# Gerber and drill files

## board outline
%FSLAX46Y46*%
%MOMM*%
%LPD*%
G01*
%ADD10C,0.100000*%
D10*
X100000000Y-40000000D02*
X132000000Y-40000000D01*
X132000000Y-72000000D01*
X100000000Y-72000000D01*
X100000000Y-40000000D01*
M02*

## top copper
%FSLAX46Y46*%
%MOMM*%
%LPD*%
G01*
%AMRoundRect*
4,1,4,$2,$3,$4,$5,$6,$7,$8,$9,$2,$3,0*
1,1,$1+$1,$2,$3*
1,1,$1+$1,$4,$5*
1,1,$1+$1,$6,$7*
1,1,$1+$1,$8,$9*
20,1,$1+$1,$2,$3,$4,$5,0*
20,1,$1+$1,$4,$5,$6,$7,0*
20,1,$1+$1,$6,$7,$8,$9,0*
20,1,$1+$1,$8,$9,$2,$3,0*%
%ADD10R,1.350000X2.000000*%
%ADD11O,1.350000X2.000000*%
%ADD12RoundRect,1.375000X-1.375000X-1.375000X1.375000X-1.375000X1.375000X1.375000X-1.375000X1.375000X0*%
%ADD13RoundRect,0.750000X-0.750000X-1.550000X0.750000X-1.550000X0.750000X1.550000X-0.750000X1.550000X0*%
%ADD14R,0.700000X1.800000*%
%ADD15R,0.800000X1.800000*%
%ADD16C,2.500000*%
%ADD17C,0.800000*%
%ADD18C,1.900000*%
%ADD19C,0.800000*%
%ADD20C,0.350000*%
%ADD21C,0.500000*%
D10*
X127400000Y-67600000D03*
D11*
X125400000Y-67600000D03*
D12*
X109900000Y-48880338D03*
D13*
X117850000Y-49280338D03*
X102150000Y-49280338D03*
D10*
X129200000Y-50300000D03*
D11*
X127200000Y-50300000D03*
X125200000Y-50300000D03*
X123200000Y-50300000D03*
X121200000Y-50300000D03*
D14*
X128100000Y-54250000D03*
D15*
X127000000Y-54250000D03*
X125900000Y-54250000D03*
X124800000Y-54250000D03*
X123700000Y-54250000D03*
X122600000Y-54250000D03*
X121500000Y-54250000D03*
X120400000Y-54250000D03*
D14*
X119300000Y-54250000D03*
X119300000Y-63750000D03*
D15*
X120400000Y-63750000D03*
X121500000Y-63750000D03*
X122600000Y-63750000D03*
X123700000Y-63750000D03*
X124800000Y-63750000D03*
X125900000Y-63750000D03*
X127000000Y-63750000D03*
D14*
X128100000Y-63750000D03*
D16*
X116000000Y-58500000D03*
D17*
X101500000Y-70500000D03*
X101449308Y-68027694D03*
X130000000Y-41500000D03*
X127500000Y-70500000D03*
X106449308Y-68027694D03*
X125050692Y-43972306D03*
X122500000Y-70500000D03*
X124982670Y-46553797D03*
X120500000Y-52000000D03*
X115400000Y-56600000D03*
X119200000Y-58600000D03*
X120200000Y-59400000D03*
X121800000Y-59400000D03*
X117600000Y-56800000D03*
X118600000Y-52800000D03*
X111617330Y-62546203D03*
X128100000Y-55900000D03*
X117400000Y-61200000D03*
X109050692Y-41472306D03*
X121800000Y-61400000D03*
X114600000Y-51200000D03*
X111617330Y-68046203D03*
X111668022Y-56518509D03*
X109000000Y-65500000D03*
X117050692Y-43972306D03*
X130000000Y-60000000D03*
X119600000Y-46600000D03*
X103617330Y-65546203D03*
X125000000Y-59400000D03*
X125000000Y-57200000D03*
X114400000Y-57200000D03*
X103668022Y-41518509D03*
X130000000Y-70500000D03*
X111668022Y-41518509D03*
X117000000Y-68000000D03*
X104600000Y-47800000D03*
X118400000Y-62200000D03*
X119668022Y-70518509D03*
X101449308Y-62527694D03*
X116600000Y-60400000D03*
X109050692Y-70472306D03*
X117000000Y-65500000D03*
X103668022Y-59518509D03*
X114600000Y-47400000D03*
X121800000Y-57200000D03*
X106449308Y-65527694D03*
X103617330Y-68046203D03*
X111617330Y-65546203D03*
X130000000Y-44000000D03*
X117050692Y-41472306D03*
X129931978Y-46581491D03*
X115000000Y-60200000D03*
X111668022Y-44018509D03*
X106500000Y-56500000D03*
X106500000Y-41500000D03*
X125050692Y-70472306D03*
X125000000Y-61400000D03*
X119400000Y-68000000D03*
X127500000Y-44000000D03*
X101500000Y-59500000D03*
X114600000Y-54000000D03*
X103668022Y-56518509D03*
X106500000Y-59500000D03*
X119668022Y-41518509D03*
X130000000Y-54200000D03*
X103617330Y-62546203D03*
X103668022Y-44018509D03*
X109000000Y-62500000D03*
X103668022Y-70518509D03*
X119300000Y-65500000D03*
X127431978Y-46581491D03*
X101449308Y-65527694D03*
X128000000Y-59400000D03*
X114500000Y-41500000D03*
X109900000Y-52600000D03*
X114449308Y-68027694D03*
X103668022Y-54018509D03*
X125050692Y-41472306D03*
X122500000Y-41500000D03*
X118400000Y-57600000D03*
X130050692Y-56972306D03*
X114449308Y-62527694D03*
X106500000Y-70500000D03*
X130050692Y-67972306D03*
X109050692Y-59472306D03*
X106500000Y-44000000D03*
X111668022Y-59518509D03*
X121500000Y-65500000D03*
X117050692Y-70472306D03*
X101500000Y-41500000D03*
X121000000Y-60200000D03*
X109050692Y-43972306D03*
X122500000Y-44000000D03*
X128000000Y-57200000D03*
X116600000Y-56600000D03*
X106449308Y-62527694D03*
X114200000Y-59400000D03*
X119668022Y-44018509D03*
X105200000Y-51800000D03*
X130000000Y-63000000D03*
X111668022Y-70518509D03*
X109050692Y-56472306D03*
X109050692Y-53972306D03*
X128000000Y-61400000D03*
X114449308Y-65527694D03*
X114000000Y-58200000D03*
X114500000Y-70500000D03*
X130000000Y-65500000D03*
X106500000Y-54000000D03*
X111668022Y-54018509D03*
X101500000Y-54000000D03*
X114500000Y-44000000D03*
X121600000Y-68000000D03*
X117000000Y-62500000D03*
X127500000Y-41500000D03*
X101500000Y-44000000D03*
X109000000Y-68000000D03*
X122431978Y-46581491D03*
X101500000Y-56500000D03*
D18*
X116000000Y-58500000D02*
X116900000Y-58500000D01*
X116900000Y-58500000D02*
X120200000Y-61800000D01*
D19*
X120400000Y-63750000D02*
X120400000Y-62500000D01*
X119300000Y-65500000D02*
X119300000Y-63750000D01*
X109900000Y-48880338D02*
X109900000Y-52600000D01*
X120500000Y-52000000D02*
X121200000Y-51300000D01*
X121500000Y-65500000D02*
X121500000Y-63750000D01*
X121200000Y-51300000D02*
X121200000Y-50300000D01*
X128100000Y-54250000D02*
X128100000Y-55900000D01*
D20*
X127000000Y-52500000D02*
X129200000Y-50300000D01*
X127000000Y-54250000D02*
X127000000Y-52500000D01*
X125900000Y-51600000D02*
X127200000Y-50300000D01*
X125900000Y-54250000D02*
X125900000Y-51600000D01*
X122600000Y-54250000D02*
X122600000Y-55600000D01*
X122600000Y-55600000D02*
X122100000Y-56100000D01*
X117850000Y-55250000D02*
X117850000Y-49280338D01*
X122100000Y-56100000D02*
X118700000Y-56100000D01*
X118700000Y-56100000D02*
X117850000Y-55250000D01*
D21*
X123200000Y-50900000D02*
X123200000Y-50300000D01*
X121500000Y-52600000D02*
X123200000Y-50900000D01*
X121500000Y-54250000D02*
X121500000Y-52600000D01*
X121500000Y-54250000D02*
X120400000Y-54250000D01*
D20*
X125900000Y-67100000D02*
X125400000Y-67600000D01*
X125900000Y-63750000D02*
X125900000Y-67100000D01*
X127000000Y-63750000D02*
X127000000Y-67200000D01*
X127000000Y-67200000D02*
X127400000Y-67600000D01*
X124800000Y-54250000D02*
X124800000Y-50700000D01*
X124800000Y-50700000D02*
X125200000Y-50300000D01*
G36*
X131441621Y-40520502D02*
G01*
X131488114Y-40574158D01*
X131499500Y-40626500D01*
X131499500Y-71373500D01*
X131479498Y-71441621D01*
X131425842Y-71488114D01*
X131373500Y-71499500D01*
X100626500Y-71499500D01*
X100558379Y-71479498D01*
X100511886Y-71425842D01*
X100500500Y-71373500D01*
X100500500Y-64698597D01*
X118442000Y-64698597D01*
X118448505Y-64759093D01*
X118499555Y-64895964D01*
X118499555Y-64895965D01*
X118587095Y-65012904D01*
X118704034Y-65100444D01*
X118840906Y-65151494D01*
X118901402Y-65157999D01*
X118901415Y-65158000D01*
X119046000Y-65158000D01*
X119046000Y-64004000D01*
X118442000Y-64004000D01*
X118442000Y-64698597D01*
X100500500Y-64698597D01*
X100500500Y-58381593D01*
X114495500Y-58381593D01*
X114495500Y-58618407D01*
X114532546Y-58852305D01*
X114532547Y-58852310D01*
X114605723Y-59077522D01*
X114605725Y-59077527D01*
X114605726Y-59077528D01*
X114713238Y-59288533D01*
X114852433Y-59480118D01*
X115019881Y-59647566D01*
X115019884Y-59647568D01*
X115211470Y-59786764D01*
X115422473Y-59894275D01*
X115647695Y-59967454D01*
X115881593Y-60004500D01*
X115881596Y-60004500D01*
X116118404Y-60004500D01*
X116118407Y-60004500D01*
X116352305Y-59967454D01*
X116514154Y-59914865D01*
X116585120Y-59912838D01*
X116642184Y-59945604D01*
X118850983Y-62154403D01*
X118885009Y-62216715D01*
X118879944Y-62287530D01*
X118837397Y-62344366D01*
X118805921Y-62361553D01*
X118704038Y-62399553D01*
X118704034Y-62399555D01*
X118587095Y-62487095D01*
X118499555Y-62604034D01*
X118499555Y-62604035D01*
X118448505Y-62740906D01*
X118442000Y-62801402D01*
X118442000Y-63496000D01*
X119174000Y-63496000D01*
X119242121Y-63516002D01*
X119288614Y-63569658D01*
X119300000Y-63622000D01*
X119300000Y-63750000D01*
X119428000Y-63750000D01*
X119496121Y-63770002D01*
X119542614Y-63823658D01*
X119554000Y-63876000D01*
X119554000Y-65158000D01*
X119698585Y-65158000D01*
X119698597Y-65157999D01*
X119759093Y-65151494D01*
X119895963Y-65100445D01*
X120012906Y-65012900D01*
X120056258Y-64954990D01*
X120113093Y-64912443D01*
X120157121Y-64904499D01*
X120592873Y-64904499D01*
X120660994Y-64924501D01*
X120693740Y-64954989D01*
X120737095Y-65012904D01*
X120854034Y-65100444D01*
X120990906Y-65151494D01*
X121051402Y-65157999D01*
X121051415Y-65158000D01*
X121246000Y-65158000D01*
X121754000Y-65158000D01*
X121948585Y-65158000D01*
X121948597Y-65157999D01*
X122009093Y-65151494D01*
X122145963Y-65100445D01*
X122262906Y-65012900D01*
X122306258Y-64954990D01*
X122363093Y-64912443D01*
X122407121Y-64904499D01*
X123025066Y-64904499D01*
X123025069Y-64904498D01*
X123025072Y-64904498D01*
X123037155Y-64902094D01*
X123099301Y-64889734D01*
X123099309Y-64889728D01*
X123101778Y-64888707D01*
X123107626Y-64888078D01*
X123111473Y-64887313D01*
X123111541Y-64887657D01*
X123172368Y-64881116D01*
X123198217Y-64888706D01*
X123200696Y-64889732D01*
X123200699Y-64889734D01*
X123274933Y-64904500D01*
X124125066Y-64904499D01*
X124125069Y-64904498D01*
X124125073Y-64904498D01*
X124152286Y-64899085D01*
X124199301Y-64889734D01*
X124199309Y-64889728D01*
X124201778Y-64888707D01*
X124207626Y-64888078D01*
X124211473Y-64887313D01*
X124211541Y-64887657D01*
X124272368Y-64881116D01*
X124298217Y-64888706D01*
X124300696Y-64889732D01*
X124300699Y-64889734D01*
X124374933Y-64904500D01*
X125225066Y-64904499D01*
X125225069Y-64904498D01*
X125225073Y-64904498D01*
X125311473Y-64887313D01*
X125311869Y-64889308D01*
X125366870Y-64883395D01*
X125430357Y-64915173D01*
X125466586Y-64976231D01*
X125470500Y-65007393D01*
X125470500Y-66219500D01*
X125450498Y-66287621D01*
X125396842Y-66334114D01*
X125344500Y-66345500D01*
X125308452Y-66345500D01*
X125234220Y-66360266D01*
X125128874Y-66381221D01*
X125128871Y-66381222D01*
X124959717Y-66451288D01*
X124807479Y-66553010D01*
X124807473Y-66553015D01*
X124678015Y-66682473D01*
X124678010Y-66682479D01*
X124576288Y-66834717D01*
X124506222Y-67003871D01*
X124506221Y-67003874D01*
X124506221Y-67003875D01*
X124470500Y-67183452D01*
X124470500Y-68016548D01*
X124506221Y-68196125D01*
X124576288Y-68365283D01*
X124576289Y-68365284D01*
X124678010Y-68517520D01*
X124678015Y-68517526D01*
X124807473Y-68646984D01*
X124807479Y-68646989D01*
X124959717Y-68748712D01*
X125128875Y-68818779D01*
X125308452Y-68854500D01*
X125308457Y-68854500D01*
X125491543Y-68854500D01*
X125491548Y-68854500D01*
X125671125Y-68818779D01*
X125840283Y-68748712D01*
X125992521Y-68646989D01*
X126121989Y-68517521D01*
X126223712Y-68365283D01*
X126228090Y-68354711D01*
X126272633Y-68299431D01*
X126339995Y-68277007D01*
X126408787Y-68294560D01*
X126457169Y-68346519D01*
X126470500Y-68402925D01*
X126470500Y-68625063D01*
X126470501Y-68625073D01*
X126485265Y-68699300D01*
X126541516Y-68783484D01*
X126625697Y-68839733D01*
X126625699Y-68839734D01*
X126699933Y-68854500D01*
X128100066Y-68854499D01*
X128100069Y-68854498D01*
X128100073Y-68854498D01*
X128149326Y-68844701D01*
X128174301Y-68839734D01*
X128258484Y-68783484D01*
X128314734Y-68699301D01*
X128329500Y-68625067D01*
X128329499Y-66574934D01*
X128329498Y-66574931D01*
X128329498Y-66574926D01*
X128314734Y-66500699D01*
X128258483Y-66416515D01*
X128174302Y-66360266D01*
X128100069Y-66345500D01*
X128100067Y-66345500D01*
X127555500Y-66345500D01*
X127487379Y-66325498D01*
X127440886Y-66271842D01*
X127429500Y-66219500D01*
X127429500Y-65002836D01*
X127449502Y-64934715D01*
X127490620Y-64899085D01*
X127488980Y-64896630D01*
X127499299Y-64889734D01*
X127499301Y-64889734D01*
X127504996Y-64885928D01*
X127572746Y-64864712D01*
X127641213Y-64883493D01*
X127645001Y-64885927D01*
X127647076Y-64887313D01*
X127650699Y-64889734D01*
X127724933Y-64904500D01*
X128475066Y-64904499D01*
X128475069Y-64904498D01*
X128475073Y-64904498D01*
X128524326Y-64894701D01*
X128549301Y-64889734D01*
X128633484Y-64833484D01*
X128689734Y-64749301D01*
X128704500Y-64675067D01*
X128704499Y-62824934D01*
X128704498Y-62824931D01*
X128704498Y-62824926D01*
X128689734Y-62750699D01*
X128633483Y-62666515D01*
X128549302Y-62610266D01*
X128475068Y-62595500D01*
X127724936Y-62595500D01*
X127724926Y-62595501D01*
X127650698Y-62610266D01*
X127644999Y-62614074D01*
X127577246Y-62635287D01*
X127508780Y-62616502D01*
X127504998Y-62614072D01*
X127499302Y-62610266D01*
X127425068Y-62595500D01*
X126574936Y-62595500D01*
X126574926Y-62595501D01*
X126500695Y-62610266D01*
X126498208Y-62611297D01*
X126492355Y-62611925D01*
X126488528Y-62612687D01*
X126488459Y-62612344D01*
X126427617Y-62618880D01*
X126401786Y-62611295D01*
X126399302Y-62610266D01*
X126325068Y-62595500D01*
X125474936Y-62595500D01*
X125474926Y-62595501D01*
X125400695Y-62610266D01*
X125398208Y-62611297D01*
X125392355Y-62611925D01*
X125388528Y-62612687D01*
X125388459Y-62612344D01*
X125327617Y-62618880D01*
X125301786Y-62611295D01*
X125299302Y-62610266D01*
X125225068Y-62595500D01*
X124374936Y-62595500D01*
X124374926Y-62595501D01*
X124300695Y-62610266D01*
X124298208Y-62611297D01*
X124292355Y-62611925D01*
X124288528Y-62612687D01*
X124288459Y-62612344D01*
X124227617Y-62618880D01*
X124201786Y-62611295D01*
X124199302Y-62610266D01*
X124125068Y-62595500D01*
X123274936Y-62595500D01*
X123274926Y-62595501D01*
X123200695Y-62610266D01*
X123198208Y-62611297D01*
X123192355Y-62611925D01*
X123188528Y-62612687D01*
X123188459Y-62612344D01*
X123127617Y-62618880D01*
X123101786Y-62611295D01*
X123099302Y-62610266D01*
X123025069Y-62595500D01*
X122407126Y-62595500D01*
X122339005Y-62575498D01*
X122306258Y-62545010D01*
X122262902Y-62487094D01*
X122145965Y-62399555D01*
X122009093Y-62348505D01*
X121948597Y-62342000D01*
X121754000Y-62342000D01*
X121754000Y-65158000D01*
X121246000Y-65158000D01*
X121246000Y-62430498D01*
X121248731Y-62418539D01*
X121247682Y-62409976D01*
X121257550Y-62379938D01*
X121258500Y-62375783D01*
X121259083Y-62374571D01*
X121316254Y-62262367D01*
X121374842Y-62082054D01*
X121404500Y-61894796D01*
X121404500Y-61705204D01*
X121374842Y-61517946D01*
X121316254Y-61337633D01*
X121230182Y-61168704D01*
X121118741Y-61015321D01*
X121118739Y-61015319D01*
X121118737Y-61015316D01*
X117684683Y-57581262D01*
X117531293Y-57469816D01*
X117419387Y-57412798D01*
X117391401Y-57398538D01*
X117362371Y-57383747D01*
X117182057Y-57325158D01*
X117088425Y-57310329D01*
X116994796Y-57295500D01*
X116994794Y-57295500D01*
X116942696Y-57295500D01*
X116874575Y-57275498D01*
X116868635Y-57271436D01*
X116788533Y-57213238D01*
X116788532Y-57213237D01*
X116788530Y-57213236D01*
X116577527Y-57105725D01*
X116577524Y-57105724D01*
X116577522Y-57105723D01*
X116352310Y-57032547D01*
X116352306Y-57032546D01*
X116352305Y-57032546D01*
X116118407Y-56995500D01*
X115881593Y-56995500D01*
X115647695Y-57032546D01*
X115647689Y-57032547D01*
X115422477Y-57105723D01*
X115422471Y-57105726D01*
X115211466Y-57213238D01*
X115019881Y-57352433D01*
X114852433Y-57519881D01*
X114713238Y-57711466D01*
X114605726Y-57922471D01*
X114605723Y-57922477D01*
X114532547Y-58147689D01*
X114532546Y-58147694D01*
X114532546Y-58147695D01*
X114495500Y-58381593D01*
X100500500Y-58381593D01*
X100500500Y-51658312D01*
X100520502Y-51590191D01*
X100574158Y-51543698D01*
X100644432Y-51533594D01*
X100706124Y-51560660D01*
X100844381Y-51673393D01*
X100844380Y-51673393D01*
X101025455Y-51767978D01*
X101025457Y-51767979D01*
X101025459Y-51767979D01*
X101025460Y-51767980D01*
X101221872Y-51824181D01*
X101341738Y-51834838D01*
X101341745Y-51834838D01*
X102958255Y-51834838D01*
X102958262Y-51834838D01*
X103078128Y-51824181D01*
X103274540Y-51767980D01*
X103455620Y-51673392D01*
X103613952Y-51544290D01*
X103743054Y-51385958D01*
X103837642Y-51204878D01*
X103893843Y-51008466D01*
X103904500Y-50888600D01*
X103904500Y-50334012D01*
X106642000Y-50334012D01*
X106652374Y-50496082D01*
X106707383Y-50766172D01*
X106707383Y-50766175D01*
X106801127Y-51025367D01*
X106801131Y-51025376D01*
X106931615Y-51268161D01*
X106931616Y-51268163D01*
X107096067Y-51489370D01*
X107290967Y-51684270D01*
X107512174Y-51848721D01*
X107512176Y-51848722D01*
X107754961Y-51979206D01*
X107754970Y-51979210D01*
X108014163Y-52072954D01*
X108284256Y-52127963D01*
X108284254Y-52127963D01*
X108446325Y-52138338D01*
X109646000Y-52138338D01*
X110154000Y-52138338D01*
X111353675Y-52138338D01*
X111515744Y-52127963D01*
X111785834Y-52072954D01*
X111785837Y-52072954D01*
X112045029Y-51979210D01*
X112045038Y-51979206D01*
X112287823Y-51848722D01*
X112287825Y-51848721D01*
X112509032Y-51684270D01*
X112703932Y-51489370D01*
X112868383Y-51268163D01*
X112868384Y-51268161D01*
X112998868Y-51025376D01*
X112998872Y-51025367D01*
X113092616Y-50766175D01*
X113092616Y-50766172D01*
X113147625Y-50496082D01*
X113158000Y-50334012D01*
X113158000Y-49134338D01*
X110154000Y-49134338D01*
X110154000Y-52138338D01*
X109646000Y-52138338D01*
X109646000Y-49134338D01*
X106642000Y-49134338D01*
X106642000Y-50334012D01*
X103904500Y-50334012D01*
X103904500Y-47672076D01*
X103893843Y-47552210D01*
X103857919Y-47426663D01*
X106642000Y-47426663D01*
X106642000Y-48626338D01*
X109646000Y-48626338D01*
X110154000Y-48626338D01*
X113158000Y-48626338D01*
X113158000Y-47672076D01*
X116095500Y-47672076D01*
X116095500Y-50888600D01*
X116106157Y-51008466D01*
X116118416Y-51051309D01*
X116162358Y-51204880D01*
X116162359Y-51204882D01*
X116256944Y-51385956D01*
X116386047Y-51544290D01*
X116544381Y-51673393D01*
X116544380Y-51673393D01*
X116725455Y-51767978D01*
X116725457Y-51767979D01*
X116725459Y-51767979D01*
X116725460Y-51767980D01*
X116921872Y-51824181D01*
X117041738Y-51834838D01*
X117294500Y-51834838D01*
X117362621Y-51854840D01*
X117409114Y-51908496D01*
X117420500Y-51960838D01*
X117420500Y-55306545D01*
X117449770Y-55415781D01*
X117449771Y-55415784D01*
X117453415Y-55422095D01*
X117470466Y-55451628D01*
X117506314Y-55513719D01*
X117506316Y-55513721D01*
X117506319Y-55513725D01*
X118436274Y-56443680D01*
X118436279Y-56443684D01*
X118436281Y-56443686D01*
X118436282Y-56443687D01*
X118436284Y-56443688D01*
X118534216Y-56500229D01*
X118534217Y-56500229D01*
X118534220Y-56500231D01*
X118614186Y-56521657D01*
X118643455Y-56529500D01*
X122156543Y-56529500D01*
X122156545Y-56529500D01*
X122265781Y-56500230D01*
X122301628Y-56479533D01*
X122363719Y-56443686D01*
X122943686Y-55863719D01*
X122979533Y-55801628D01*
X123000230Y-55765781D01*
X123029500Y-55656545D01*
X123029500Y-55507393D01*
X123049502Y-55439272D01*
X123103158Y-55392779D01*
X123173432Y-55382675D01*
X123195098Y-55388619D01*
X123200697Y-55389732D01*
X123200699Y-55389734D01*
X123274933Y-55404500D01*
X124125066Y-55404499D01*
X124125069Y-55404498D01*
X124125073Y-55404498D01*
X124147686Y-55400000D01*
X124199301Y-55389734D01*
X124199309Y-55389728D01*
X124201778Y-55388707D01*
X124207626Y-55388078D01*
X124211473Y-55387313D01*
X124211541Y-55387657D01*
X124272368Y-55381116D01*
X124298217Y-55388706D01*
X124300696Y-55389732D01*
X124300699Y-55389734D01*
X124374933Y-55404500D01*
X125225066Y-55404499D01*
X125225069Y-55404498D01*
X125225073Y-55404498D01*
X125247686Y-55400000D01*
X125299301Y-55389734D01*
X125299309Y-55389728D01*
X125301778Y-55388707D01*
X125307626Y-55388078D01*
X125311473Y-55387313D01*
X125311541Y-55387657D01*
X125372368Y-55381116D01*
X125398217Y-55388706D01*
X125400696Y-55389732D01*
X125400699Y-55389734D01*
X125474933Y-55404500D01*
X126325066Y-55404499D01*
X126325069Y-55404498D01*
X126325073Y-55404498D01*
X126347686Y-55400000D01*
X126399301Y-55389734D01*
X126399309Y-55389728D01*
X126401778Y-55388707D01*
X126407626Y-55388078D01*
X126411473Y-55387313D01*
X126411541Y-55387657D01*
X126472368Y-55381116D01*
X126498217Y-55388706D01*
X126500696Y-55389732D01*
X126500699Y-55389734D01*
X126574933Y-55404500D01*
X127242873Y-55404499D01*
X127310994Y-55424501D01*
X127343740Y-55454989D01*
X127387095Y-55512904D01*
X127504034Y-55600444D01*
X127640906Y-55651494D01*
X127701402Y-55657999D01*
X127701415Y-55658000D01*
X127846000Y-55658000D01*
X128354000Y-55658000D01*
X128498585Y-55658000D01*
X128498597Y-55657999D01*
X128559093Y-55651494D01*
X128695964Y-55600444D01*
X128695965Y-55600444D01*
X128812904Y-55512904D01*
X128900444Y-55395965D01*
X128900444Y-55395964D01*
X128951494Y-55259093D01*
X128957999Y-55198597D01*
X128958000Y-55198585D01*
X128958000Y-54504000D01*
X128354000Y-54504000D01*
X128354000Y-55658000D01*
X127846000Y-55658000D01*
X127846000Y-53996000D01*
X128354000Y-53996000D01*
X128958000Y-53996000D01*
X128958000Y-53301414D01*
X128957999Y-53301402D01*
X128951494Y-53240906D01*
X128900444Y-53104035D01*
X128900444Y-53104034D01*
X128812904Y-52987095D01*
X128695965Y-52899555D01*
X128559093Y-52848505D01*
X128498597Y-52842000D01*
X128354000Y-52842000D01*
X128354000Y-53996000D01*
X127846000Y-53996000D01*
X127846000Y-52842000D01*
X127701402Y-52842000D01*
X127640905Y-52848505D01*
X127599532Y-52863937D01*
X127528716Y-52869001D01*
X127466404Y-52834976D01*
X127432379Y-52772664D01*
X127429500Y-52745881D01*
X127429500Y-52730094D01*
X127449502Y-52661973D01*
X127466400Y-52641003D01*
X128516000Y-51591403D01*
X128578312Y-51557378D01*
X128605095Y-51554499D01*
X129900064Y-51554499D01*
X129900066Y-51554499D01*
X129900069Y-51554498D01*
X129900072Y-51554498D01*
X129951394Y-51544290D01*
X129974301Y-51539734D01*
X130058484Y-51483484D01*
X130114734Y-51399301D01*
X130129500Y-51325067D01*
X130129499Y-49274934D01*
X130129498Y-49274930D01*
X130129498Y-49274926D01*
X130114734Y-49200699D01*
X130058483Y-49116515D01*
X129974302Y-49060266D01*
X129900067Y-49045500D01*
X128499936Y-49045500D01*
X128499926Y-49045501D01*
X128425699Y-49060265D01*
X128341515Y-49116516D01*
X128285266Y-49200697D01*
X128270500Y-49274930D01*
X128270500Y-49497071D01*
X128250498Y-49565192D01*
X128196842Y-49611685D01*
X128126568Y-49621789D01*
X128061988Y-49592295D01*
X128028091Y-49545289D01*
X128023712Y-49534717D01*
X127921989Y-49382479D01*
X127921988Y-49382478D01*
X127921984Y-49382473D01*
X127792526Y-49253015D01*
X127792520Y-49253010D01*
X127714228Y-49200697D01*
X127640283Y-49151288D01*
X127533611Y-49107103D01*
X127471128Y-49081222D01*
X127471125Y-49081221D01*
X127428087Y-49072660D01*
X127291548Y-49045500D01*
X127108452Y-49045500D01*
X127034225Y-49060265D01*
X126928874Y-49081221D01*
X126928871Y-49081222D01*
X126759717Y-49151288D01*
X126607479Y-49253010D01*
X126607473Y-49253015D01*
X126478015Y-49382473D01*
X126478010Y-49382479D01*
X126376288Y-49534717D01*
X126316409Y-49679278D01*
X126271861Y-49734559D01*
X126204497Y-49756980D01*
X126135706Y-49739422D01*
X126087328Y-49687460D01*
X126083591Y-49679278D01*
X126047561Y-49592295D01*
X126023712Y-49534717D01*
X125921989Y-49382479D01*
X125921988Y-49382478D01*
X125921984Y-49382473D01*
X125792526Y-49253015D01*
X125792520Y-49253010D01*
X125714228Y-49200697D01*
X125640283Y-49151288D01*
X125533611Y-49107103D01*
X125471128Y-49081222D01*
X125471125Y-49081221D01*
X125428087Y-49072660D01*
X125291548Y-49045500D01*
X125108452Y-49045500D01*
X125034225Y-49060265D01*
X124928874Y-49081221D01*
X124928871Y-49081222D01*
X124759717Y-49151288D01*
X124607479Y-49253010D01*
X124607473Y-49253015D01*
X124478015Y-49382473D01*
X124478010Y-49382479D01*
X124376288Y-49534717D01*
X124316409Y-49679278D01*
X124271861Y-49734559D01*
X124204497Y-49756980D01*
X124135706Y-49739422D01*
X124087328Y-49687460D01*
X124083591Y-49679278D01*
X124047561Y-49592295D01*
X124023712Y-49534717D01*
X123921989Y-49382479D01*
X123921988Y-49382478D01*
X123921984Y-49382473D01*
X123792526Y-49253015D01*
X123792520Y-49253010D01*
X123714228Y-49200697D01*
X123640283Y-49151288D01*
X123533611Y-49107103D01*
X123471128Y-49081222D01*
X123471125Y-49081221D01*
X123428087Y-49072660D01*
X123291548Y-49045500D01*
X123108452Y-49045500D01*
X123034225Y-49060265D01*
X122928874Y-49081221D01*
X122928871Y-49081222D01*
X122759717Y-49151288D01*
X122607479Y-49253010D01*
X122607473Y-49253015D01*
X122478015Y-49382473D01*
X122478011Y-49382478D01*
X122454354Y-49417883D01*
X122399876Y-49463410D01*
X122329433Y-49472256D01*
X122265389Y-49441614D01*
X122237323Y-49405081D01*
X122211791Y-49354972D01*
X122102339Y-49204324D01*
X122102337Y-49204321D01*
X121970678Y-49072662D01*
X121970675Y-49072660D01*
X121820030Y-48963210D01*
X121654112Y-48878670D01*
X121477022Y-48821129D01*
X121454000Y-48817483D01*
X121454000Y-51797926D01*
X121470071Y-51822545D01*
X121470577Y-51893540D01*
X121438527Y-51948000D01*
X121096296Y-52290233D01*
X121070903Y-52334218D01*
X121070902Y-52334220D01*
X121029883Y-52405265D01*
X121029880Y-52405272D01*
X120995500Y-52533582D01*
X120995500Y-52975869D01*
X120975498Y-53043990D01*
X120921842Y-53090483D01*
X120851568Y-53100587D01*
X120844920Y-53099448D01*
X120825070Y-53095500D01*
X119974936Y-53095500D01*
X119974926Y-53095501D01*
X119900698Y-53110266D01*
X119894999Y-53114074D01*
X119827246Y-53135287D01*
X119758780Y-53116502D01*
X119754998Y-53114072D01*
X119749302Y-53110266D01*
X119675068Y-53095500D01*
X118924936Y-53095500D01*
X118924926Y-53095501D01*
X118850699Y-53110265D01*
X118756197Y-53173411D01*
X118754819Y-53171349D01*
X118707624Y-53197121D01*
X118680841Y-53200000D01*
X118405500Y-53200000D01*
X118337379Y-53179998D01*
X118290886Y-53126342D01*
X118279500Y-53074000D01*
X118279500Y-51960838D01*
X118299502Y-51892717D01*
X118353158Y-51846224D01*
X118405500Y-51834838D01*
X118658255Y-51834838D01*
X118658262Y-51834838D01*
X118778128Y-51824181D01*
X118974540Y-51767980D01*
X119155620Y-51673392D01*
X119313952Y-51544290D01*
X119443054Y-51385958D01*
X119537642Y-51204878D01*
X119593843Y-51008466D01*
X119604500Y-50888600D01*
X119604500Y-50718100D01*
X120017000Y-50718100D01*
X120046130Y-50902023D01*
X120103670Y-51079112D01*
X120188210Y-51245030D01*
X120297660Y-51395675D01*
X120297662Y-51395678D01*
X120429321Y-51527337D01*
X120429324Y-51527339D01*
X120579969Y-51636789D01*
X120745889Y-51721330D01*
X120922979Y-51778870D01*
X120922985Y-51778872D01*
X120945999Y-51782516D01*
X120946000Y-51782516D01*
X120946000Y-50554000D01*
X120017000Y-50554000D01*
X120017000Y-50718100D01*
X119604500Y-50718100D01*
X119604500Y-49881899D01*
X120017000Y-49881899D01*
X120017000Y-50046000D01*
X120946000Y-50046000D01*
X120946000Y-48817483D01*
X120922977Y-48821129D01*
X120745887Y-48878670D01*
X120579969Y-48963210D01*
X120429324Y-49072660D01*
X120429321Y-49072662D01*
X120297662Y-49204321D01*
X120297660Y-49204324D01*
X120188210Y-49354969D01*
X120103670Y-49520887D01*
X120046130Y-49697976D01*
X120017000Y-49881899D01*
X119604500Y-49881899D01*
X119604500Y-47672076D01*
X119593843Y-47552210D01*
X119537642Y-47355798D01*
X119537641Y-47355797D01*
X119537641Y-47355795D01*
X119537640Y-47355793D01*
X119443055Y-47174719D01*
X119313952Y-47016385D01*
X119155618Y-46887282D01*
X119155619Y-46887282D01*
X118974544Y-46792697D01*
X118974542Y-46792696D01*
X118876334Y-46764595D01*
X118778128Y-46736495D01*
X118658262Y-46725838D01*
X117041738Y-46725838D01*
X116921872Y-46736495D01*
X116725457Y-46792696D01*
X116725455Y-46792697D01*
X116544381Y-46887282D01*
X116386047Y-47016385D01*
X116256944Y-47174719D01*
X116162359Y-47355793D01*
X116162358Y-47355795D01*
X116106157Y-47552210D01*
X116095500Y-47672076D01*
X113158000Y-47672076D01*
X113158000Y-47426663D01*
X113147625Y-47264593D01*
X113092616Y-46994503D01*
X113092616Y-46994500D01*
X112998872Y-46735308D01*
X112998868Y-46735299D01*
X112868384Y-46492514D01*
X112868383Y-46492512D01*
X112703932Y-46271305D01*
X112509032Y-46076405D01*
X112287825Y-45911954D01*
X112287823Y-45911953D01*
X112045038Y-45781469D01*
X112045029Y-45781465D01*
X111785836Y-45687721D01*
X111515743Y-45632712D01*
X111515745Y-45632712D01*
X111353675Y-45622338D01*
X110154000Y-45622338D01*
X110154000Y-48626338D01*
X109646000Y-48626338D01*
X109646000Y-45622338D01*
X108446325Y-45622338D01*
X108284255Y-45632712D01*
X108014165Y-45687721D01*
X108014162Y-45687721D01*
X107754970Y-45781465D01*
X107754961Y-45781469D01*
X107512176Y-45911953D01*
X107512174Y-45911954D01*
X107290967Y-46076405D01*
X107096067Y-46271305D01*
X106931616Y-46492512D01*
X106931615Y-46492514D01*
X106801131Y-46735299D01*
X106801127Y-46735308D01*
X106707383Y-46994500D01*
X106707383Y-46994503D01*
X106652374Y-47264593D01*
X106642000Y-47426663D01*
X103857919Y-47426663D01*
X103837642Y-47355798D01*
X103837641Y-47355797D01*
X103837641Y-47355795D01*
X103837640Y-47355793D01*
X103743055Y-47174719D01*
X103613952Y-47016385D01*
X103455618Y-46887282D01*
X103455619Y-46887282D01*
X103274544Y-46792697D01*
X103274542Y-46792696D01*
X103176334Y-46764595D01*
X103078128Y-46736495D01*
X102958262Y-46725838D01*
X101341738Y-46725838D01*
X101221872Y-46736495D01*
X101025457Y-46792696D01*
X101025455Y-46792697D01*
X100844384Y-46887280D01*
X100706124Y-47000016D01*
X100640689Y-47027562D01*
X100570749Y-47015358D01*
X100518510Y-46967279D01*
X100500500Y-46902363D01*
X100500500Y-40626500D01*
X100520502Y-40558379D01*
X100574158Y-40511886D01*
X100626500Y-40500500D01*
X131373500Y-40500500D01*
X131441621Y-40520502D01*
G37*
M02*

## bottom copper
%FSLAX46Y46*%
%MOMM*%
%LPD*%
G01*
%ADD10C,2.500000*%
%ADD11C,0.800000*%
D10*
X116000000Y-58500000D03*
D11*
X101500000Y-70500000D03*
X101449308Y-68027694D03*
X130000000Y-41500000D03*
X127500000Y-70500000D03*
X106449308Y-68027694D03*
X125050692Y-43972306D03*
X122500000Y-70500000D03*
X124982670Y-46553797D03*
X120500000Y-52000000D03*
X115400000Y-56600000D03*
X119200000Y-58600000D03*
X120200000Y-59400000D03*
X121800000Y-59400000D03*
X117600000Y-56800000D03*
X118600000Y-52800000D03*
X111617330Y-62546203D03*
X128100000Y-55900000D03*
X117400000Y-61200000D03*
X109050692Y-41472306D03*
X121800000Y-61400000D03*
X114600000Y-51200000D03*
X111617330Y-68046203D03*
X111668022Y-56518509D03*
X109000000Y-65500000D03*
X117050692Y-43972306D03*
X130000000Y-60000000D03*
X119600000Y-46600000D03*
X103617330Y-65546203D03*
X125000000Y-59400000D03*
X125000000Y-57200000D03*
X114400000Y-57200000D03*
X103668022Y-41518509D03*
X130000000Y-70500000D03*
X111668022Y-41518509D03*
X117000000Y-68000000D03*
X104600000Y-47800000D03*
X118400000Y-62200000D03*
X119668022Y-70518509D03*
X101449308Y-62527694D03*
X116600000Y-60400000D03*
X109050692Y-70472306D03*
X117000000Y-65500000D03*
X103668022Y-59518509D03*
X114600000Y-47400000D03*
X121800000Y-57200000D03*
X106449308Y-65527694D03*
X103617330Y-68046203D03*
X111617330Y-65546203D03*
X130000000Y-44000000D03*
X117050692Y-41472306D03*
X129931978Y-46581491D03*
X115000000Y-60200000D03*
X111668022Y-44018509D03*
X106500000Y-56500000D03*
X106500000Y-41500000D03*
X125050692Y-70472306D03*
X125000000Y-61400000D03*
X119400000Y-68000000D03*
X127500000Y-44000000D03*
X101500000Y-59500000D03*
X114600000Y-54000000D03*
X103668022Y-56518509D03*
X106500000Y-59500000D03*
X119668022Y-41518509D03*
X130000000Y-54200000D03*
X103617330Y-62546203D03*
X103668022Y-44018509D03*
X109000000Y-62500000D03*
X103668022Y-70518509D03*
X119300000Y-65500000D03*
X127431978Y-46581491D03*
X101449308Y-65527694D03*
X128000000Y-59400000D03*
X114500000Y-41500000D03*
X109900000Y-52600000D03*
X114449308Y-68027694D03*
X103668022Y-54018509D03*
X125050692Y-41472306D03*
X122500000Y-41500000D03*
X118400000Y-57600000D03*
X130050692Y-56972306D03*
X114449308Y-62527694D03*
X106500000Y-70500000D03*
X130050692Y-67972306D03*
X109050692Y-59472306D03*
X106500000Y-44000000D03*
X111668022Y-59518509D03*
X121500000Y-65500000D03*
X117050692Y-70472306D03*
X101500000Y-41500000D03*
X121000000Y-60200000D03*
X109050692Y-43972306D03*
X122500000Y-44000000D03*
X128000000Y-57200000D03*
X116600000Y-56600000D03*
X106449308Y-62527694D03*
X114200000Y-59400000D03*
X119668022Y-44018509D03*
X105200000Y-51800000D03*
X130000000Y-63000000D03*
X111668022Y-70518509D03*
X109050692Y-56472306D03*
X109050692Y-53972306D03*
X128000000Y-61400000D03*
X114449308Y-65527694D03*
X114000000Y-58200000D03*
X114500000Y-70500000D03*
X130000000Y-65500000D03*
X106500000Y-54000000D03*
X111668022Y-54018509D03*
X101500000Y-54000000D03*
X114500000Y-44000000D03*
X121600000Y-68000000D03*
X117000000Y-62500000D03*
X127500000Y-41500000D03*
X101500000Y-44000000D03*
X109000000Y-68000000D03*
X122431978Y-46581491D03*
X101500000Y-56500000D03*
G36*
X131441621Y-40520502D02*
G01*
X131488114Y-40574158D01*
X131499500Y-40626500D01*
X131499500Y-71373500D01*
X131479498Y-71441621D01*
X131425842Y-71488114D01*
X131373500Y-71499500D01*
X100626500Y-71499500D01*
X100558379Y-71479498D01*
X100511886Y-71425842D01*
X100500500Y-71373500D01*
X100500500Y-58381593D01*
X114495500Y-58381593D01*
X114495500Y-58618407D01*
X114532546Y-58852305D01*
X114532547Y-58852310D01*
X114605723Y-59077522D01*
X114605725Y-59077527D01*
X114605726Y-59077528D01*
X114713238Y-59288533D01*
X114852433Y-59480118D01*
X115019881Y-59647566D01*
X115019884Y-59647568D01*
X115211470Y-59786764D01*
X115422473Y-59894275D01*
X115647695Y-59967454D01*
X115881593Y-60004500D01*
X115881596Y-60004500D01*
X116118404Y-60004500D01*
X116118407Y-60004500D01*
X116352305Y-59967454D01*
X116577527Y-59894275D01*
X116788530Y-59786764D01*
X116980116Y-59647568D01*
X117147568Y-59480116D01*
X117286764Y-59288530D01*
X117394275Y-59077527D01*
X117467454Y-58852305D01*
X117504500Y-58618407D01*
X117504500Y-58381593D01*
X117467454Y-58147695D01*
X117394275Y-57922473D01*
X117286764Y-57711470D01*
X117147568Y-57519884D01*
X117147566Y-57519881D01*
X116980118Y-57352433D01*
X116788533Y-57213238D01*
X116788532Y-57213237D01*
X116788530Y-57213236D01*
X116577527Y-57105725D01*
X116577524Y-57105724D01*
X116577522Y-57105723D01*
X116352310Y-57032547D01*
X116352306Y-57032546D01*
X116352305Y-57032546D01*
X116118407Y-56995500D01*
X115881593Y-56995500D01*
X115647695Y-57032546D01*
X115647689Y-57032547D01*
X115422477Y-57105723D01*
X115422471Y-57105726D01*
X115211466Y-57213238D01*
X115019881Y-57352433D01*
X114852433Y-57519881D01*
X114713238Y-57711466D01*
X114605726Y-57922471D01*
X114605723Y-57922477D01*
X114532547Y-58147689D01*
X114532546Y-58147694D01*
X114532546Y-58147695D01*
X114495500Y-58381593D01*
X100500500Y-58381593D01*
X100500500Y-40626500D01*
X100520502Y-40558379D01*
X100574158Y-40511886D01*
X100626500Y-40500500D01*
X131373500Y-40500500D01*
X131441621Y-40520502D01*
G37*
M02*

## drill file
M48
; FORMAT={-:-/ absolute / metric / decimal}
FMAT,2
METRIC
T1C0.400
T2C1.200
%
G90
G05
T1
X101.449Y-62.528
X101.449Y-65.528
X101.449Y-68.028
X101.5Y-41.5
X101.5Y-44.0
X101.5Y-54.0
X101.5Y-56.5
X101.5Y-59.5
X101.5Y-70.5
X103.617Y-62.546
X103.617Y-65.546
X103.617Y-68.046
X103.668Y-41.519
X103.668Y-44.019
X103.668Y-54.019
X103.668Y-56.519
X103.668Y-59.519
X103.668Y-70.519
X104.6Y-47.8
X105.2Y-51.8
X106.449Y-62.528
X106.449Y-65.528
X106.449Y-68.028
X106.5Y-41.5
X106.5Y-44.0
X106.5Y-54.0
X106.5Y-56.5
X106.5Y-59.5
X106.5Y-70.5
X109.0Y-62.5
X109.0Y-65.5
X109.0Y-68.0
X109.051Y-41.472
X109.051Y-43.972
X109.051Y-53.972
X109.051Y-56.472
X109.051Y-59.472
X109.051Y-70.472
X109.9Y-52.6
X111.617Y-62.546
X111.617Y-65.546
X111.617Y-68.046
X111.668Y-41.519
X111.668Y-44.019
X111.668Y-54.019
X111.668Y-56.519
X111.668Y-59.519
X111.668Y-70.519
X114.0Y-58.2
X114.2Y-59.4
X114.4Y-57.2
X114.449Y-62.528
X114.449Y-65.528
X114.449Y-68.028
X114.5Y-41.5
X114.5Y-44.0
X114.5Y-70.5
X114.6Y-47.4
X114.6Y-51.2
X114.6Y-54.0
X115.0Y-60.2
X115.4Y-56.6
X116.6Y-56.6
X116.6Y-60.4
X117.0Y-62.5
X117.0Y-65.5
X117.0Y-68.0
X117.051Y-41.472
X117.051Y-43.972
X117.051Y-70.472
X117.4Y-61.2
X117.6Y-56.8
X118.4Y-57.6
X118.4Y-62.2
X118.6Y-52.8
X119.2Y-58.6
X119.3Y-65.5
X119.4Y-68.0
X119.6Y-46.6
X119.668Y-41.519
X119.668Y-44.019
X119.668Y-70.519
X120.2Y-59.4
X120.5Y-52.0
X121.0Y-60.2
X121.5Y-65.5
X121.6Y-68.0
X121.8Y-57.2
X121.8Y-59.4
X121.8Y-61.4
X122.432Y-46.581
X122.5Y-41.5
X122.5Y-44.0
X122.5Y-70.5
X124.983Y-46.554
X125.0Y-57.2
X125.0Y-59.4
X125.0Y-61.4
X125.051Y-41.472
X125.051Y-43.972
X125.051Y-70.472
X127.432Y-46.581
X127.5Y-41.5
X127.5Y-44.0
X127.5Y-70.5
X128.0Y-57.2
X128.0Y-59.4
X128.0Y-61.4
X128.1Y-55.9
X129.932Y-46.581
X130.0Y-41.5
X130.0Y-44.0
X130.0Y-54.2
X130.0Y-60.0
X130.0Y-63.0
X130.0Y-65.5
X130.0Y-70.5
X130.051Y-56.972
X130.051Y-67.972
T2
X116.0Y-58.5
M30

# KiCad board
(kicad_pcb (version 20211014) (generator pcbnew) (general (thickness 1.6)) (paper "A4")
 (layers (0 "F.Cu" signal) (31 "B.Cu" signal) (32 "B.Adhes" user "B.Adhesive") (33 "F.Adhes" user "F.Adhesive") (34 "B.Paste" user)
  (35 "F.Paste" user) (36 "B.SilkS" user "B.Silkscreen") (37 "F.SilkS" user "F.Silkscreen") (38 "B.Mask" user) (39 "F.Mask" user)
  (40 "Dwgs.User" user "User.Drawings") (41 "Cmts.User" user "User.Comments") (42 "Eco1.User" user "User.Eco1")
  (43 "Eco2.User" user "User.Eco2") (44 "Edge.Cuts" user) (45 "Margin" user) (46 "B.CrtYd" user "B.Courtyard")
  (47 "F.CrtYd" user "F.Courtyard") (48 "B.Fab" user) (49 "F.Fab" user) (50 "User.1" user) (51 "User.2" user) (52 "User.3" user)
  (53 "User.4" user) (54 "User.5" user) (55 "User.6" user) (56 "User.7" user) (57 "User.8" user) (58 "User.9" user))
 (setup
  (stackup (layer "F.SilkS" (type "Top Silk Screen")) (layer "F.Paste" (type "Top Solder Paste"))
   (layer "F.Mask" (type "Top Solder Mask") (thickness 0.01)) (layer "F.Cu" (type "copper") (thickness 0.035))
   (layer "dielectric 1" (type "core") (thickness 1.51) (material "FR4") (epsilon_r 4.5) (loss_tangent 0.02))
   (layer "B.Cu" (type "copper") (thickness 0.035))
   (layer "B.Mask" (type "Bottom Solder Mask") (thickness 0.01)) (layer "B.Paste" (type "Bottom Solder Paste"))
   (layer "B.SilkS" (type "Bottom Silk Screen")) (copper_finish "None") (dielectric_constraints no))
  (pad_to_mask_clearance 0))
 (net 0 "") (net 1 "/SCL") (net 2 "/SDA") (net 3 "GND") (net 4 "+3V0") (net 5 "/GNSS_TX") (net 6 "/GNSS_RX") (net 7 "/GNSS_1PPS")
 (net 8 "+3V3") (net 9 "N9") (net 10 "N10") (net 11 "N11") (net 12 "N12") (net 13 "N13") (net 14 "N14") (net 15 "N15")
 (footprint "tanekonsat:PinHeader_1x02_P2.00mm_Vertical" (layer "F.Cu") (at 127.4 67.6 -90)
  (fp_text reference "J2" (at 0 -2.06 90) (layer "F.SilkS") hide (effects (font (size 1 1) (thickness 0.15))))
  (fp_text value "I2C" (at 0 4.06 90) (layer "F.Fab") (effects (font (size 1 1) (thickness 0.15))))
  (pad "1" smd rect (at 0 0 270) (size 2 1.35) (layers "F.Cu" "F.Paste" "F.Mask") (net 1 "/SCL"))
  (pad "2" smd oval (at 0 2 270) (size 2 1.35) (layers "F.Cu" "F.Paste" "F.Mask") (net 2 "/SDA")))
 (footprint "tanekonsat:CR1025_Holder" (layer "F.Cu") (at 103.65 54.880338)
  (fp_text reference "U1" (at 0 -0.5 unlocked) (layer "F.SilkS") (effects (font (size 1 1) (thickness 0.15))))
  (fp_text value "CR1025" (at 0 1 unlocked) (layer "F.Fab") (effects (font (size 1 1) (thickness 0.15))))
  (pad "1" smd roundrect (at 6.25 -6) (size 5.5 5.5) (layers "F.Cu" "F.Paste" "F.Mask") (roundrect_rratio 0.25) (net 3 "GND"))
  (pad "2" smd roundrect (at 14.2 -5.6) (size 3 4.6) (layers "F.Cu" "F.Paste" "F.Mask") (roundrect_rratio 0.25) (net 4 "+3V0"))
  (pad "2" smd roundrect (at -1.5 -5.6) (size 3 4.6) (layers "F.Cu" "F.Paste" "F.Mask") (roundrect_rratio 0.25) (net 4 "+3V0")))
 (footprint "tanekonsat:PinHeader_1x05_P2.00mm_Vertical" (layer "F.Cu") (at 129.2 50.3 -90)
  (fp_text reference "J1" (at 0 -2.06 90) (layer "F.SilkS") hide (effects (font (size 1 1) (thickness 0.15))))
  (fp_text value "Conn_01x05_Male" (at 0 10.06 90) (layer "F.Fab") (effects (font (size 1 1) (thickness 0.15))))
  (pad "1" smd rect (at 0 0 270) (size 2 1.35) (layers "F.Cu" "F.Paste" "F.Mask") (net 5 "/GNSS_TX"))
  (pad "2" smd oval (at 0 2 270) (size 2 1.35) (layers "F.Cu" "F.Paste" "F.Mask") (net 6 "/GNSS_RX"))
  (pad "3" smd oval (at 0 4 270) (size 2 1.35) (layers "F.Cu" "F.Paste" "F.Mask") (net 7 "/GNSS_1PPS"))
  (pad "4" smd oval (at 0 6 270) (size 2 1.35) (layers "F.Cu" "F.Paste" "F.Mask") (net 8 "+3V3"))
  (pad "5" smd oval (at 0 8 270) (size 2 1.35) (layers "F.Cu" "F.Paste" "F.Mask") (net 3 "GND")))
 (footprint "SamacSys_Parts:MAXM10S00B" (layer "F.Cu") (at 123.7 59 90)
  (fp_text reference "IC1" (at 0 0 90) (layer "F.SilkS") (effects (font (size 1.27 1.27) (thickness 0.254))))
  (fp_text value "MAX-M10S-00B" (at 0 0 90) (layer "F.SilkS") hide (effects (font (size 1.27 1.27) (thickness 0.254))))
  (pad "1" smd rect locked (at 4.75 4.4 180) (size 0.7 1.8) (layers "F.Cu" "F.Paste" "F.Mask") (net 3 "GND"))
  (pad "2" smd rect locked (at 4.75 3.3 180) (size 0.8 1.8) (layers "F.Cu" "F.Paste" "F.Mask") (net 5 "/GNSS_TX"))
  (pad "3" smd rect locked (at 4.75 2.2 180) (size 0.8 1.8) (layers "F.Cu" "F.Paste" "F.Mask") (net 6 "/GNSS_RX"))
  (pad "4" smd rect locked (at 4.75 1.1 180) (size 0.8 1.8) (layers "F.Cu" "F.Paste" "F.Mask") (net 7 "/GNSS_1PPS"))
  (pad "5" smd rect locked (at 4.75 0 180) (size 0.8 1.8) (layers "F.Cu" "F.Paste" "F.Mask") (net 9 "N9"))
  (pad "6" smd rect locked (at 4.75 -1.1 180) (size 0.8 1.8) (layers "F.Cu" "F.Paste" "F.Mask") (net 4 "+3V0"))
  (pad "7" smd rect locked (at 4.75 -2.2 180) (size 0.8 1.8) (layers "F.Cu" "F.Paste" "F.Mask") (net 8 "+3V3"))
  (pad "8" smd rect locked (at 4.75 -3.3 180) (size 0.8 1.8) (layers "F.Cu" "F.Paste" "F.Mask") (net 8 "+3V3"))
  (pad "9" smd rect locked (at 4.75 -4.4 180) (size 0.7 1.8) (layers "F.Cu" "F.Paste" "F.Mask") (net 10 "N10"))
  (pad "10" smd rect locked (at -4.75 -4.4 180) (size 0.7 1.8) (layers "F.Cu" "F.Paste" "F.Mask") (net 3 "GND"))
  (pad "11" smd rect locked (at -4.75 -3.3 180) (size 0.8 1.8) (layers "F.Cu" "F.Paste" "F.Mask") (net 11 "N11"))
  (pad "12" smd rect locked (at -4.75 -2.2 180) (size 0.8 1.8) (layers "F.Cu" "F.Paste" "F.Mask") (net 3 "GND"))
  (pad "13" smd rect locked (at -4.75 -1.1 180) (size 0.8 1.8) (layers "F.Cu" "F.Paste" "F.Mask") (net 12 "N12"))
  (pad "14" smd rect locked (at -4.75 0 180) (size 0.8 1.8) (layers "F.Cu" "F.Paste" "F.Mask") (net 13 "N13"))
  (pad "15" smd rect locked (at -4.75 1.1 180) (size 0.8 1.8) (layers "F.Cu" "F.Paste" "F.Mask") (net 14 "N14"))
  (pad "16" smd rect locked (at -4.75 2.2 180) (size 0.8 1.8) (layers "F.Cu" "F.Paste" "F.Mask") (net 2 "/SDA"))
  (pad "17" smd rect locked (at -4.75 3.3 180) (size 0.8 1.8) (layers "F.Cu" "F.Paste" "F.Mask") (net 1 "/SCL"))
  (pad "18" smd rect locked (at -4.75 4.4 180) (size 0.7 1.8) (layers "F.Cu" "F.Paste" "F.Mask") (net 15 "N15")))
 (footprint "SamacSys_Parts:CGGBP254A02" (layer "B.Cu") (at 116 58.5 180)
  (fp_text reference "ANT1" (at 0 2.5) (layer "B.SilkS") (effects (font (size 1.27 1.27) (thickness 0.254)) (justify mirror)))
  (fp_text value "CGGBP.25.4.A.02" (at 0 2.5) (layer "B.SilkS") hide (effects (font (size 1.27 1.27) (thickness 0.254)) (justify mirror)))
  (pad "1" thru_hole circle locked (at 0 0 180) (size 2.5 2.5) (drill 1.2) (layers *.Cu *.Mask) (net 11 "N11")))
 (gr_rect (start 100 40) (end 132 72) (layer "Edge.Cuts") (width 0.1) (fill none))
 (segment (start 116 58.5) (end 116.9 58.5) (width 1.9) (layer "F.Cu") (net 11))
 (segment (start 116.9 58.5) (end 120.2 61.8) (width 1.9) (layer "F.Cu") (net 11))
 (segment (start 120.4 63.75) (end 120.4 62.5) (width 0.8) (layer "F.Cu") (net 11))
 (segment (start 119.3 65.5) (end 119.3 63.75) (width 0.8) (layer "F.Cu") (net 3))
 (segment (start 109.9 48.880338) (end 109.9 52.6) (width 0.8) (layer "F.Cu") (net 3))
 (segment (start 120.5 52) (end 121.2 51.3) (width 0.8) (layer "F.Cu") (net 3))
 (segment (start 121.5 65.5) (end 121.5 63.75) (width 0.8) (layer "F.Cu") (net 3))
 (segment (start 121.2 51.3) (end 121.2 50.3) (width 0.8) (layer "F.Cu") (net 3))
 (segment (start 128.1 54.25) (end 128.1 55.9) (width 0.8) (layer "F.Cu") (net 3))
 (via (at 101.5 70.5) (size 0.8) (drill 0.4) (layers "F.Cu" "B.Cu") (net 3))
 (via (at 101.449308 68.027694) (size 0.8) (drill 0.4) (layers "F.Cu" "B.Cu") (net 3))
 (via (at 130 41.5) (size 0.8) (drill 0.4) (layers "F.Cu" "B.Cu") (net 3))
 (via (at 127.5 70.5) (size 0.8) (drill 0.4) (layers "F.Cu" "B.Cu") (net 3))
 (via (at 106.449308 68.027694) (size 0.8) (drill 0.4) (layers "F.Cu" "B.Cu") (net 3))
 (via (at 125.050692 43.972306) (size 0.8) (drill 0.4) (layers "F.Cu" "B.Cu") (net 3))
 (via (at 122.5 70.5) (size 0.8) (drill 0.4) (layers "F.Cu" "B.Cu") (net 3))
 (via (at 124.98267 46.553797) (size 0.8) (drill 0.4) (layers "F.Cu" "B.Cu") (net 3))
 (via (at 120.5 52) (size 0.8) (drill 0.4) (layers "F.Cu" "B.Cu") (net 3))
 (via (at 115.4 56.6) (size 0.8) (drill 0.4) (layers "F.Cu" "B.Cu") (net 3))
 (via (at 119.2 58.6) (size 0.8) (drill 0.4) (layers "F.Cu" "B.Cu") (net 3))
 (via (at 120.2 59.4) (size 0.8) (drill 0.4) (layers "F.Cu" "B.Cu") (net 3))
 (via (at 121.8 59.4) (size 0.8) (drill 0.4) (layers "F.Cu" "B.Cu") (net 3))
 (via (at 117.6 56.8) (size 0.8) (drill 0.4) (layers "F.Cu" "B.Cu") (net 3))
 (via (at 118.6 52.8) (size 0.8) (drill 0.4) (layers "F.Cu" "B.Cu") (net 3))
 (via (at 111.61733 62.546203) (size 0.8) (drill 0.4) (layers "F.Cu" "B.Cu") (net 3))
 (via (at 128.1 55.9) (size 0.8) (drill 0.4) (layers "F.Cu" "B.Cu") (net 3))
 (via (at 117.4 61.2) (size 0.8) (drill 0.4) (layers "F.Cu" "B.Cu") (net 3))
 (via (at 109.050692 41.472306) (size 0.8) (drill 0.4) (layers "F.Cu" "B.Cu") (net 3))
 (via (at 121.8 61.4) (size 0.8) (drill 0.4) (layers "F.Cu" "B.Cu") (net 3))
 (via (at 114.6 51.2) (size 0.8) (drill 0.4) (layers "F.Cu" "B.Cu") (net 3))
 (via (at 111.61733 68.046203) (size 0.8) (drill 0.4) (layers "F.Cu" "B.Cu") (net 3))
 (via (at 111.668022 56.518509) (size 0.8) (drill 0.4) (layers "F.Cu" "B.Cu") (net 3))
 (via (at 109 65.5) (size 0.8) (drill 0.4) (layers "F.Cu" "B.Cu") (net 3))
 (via (at 117.050692 43.972306) (size 0.8) (drill 0.4) (layers "F.Cu" "B.Cu") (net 3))
 (via (at 130 60) (size 0.8) (drill 0.4) (layers "F.Cu" "B.Cu") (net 3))
 (via (at 119.6 46.6) (size 0.8) (drill 0.4) (layers "F.Cu" "B.Cu") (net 3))
 (via (at 103.61733 65.546203) (size 0.8) (drill 0.4) (layers "F.Cu" "B.Cu") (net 3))
 (via (at 125 59.4) (size 0.8) (drill 0.4) (layers "F.Cu" "B.Cu") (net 3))
 (via (at 125 57.2) (size 0.8) (drill 0.4) (layers "F.Cu" "B.Cu") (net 3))
 (via (at 114.4 57.2) (size 0.8) (drill 0.4) (layers "F.Cu" "B.Cu") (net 3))
 (via (at 103.668022 41.518509) (size 0.8) (drill 0.4) (layers "F.Cu" "B.Cu") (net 3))
 (via (at 130 70.5) (size 0.8) (drill 0.4) (layers "F.Cu" "B.Cu") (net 3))
 (via (at 111.668022 41.518509) (size 0.8) (drill 0.4) (layers "F.Cu" "B.Cu") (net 3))
 (via (at 117 68) (size 0.8) (drill 0.4) (layers "F.Cu" "B.Cu") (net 3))
 (via (at 104.6 47.8) (size 0.8) (drill 0.4) (layers "F.Cu" "B.Cu") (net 3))
 (via (at 118.4 62.2) (size 0.8) (drill 0.4) (layers "F.Cu" "B.Cu") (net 3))
 (via (at 119.668022 70.518509) (size 0.8) (drill 0.4) (layers "F.Cu" "B.Cu") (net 3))
 (via (at 101.449308 62.527694) (size 0.8) (drill 0.4) (layers "F.Cu" "B.Cu") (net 3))
 (via (at 116.6 60.4) (size 0.8) (drill 0.4) (layers "F.Cu" "B.Cu") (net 3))
 (via (at 109.050692 70.472306) (size 0.8) (drill 0.4) (layers "F.Cu" "B.Cu") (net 3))
 (via (at 117 65.5) (size 0.8) (drill 0.4) (layers "F.Cu" "B.Cu") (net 3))
 (via (at 103.668022 59.518509) (size 0.8) (drill 0.4) (layers "F.Cu" "B.Cu") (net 3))
 (via (at 114.6 47.4) (size 0.8) (drill 0.4) (layers "F.Cu" "B.Cu") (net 3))
 (via (at 121.8 57.2) (size 0.8) (drill 0.4) (layers "F.Cu" "B.Cu") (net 3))
 (via (at 106.449308 65.527694) (size 0.8) (drill 0.4) (layers "F.Cu" "B.Cu") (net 3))
 (via (at 103.61733 68.046203) (size 0.8) (drill 0.4) (layers "F.Cu" "B.Cu") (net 3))
 (via (at 111.61733 65.546203) (size 0.8) (drill 0.4) (layers "F.Cu" "B.Cu") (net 3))
 (via (at 130 44) (size 0.8) (drill 0.4) (layers "F.Cu" "B.Cu") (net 3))
 (via (at 117.050692 41.472306) (size 0.8) (drill 0.4) (layers "F.Cu" "B.Cu") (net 3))
 (via (at 129.931978 46.581491) (size 0.8) (drill 0.4) (layers "F.Cu" "B.Cu") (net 3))
 (via (at 115 60.2) (size 0.8) (drill 0.4) (layers "F.Cu" "B.Cu") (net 3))
 (via (at 111.668022 44.018509) (size 0.8) (drill 0.4) (layers "F.Cu" "B.Cu") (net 3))
 (via (at 106.5 56.5) (size 0.8) (drill 0.4) (layers "F.Cu" "B.Cu") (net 3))
 (via (at 106.5 41.5) (size 0.8) (drill 0.4) (layers "F.Cu" "B.Cu") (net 3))
 (via (at 125.050692 70.472306) (size 0.8) (drill 0.4) (layers "F.Cu" "B.Cu") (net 3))
 (via (at 125 61.4) (size 0.8) (drill 0.4) (layers "F.Cu" "B.Cu") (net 3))
 (via (at 119.4 68) (size 0.8) (drill 0.4) (layers "F.Cu" "B.Cu") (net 3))
 (via (at 127.5 44) (size 0.8) (drill 0.4) (layers "F.Cu" "B.Cu") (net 3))
 (via (at 101.5 59.5) (size 0.8) (drill 0.4) (layers "F.Cu" "B.Cu") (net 3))
 (via (at 114.6 54) (size 0.8) (drill 0.4) (layers "F.Cu" "B.Cu") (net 3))
 (via (at 103.668022 56.518509) (size 0.8) (drill 0.4) (layers "F.Cu" "B.Cu") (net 3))
 (via (at 106.5 59.5) (size 0.8) (drill 0.4) (layers "F.Cu" "B.Cu") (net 3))
 (via (at 119.668022 41.518509) (size 0.8) (drill 0.4) (layers "F.Cu" "B.Cu") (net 3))
 (via (at 130 54.2) (size 0.8) (drill 0.4) (layers "F.Cu" "B.Cu") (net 3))
 (via (at 103.61733 62.546203) (size 0.8) (drill 0.4) (layers "F.Cu" "B.Cu") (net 3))
 (via (at 103.668022 44.018509) (size 0.8) (drill 0.4) (layers "F.Cu" "B.Cu") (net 3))
 (via (at 109 62.5) (size 0.8) (drill 0.4) (layers "F.Cu" "B.Cu") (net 3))
 (via (at 103.668022 70.518509) (size 0.8) (drill 0.4) (layers "F.Cu" "B.Cu") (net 3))
 (via (at 119.3 65.5) (size 0.8) (drill 0.4) (layers "F.Cu" "B.Cu") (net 3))
 (via (at 127.431978 46.581491) (size 0.8) (drill 0.4) (layers "F.Cu" "B.Cu") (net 3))
 (via (at 101.449308 65.527694) (size 0.8) (drill 0.4) (layers "F.Cu" "B.Cu") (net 3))
 (via (at 128 59.4) (size 0.8) (drill 0.4) (layers "F.Cu" "B.Cu") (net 3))
 (via (at 114.5 41.5) (size 0.8) (drill 0.4) (layers "F.Cu" "B.Cu") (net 3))
 (via (at 109.9 52.6) (size 0.8) (drill 0.4) (layers "F.Cu" "B.Cu") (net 3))
 (via (at 114.449308 68.027694) (size 0.8) (drill 0.4) (layers "F.Cu" "B.Cu") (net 3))
 (via (at 103.668022 54.018509) (size 0.8) (drill 0.4) (layers "F.Cu" "B.Cu") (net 3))
 (via (at 125.050692 41.472306) (size 0.8) (drill 0.4) (layers "F.Cu" "B.Cu") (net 3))
 (via (at 122.5 41.5) (size 0.8) (drill 0.4) (layers "F.Cu" "B.Cu") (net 3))
 (via (at 118.4 57.6) (size 0.8) (drill 0.4) (layers "F.Cu" "B.Cu") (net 3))
 (via (at 130.050692 56.972306) (size 0.8) (drill 0.4) (layers "F.Cu" "B.Cu") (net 3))
 (via (at 114.449308 62.527694) (size 0.8) (drill 0.4) (layers "F.Cu" "B.Cu") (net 3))
 (via (at 106.5 70.5) (size 0.8) (drill 0.4) (layers "F.Cu" "B.Cu") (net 3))
 (via (at 130.050692 67.972306) (size 0.8) (drill 0.4) (layers "F.Cu" "B.Cu") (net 3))
 (via (at 109.050692 59.472306) (size 0.8) (drill 0.4) (layers "F.Cu" "B.Cu") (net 3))
 (via (at 106.5 44) (size 0.8) (drill 0.4) (layers "F.Cu" "B.Cu") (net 3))
 (via (at 111.668022 59.518509) (size 0.8) (drill 0.4) (layers "F.Cu" "B.Cu") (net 3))
 (via (at 121.5 65.5) (size 0.8) (drill 0.4) (layers "F.Cu" "B.Cu") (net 3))
 (via (at 117.050692 70.472306) (size 0.8) (drill 0.4) (layers "F.Cu" "B.Cu") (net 3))
 (via (at 101.5 41.5) (size 0.8) (drill 0.4) (layers "F.Cu" "B.Cu") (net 3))
 (via (at 121 60.2) (size 0.8) (drill 0.4) (layers "F.Cu" "B.Cu") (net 3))
 (via (at 109.050692 43.972306) (size 0.8) (drill 0.4) (layers "F.Cu" "B.Cu") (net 3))
 (via (at 122.5 44) (size 0.8) (drill 0.4) (layers "F.Cu" "B.Cu") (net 3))
 (via (at 128 57.2) (size 0.8) (drill 0.4) (layers "F.Cu" "B.Cu") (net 3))
 (via (at 116.6 56.6) (size 0.8) (drill 0.4) (layers "F.Cu" "B.Cu") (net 3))
 (via (at 106.449308 62.527694) (size 0.8) (drill 0.4) (layers "F.Cu" "B.Cu") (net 3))
 (via (at 114.2 59.4) (size 0.8) (drill 0.4) (layers "F.Cu" "B.Cu") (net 3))
 (via (at 119.668022 44.018509) (size 0.8) (drill 0.4) (layers "F.Cu" "B.Cu") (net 3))
 (via (at 105.2 51.8) (size 0.8) (drill 0.4) (layers "F.Cu" "B.Cu") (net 3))
 (via (at 130 63) (size 0.8) (drill 0.4) (layers "F.Cu" "B.Cu") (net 3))
 (via (at 111.668022 70.518509) (size 0.8) (drill 0.4) (layers "F.Cu" "B.Cu") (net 3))
 (via (at 109.050692 56.472306) (size 0.8) (drill 0.4) (layers "F.Cu" "B.Cu") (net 3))
 (via (at 109.050692 53.972306) (size 0.8) (drill 0.4) (layers "F.Cu" "B.Cu") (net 3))
 (via (at 128 61.4) (size 0.8) (drill 0.4) (layers "F.Cu" "B.Cu") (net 3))
 (via (at 114.449308 65.527694) (size 0.8) (drill 0.4) (layers "F.Cu" "B.Cu") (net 3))
 (via (at 114 58.2) (size 0.8) (drill 0.4) (layers "F.Cu" "B.Cu") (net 3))
 (via (at 114.5 70.5) (size 0.8) (drill 0.4) (layers "F.Cu" "B.Cu") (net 3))
 (via (at 130 65.5) (size 0.8) (drill 0.4) (layers "F.Cu" "B.Cu") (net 3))
 (via (at 106.5 54) (size 0.8) (drill 0.4) (layers "F.Cu" "B.Cu") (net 3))
 (via (at 111.668022 54.018509) (size 0.8) (drill 0.4) (layers "F.Cu" "B.Cu") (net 3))
 (via (at 101.5 54) (size 0.8) (drill 0.4) (layers "F.Cu" "B.Cu") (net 3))
 (via (at 114.5 44) (size 0.8) (drill 0.4) (layers "F.Cu" "B.Cu") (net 3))
 (via (at 121.6 68) (size 0.8) (drill 0.4) (layers "F.Cu" "B.Cu") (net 3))
 (via (at 117 62.5) (size 0.8) (drill 0.4) (layers "F.Cu" "B.Cu") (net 3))
 (via (at 127.5 41.5) (size 0.8) (drill 0.4) (layers "F.Cu" "B.Cu") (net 3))
 (via (at 101.5 44) (size 0.8) (drill 0.4) (layers "F.Cu" "B.Cu") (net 3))
 (via (at 109 68) (size 0.8) (drill 0.4) (layers "F.Cu" "B.Cu") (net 3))
 (via (at 122.431978 46.581491) (size 0.8) (drill 0.4) (layers "F.Cu" "B.Cu") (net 3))
 (via (at 101.5 56.5) (size 0.8) (drill 0.4) (layers "F.Cu" "B.Cu") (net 3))
 (segment (start 127 52.5) (end 129.2 50.3) (width 0.35) (layer "F.Cu") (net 5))
 (segment (start 127 54.25) (end 127 52.5) (width 0.35) (layer "F.Cu") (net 5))
 (segment (start 125.9 51.6) (end 127.2 50.3) (width 0.35) (layer "F.Cu") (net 6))
 (segment (start 125.9 54.25) (end 125.9 51.6) (width 0.35) (layer "F.Cu") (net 6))
 (segment (start 122.6 54.25) (end 122.6 55.6) (width 0.35) (layer "F.Cu") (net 4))
 (segment (start 122.6 55.6) (end 122.1 56.1) (width 0.35) (layer "F.Cu") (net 4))
 (segment (start 117.85 55.25) (end 117.85 49.280338) (width 0.35) (layer "F.Cu") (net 4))
 (segment (start 122.1 56.1) (end 118.7 56.1) (width 0.35) (layer "F.Cu") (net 4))
 (segment (start 118.7 56.1) (end 117.85 55.25) (width 0.35) (layer "F.Cu") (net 4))
 (segment (start 123.2 50.9) (end 123.2 50.3) (width 0.5) (layer "F.Cu") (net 8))
 (segment (start 121.5 52.6) (end 123.2 50.9) (width 0.5) (layer "F.Cu") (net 8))
 (segment (start 121.5 54.25) (end 121.5 52.6) (width 0.5) (layer "F.Cu") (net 8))
 (segment (start 121.5 54.25) (end 120.4 54.25) (width 0.5) (layer "F.Cu") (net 8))
 (segment (start 125.9 67.1) (end 125.4 67.6) (width 0.35) (layer "F.Cu") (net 2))
 (segment (start 125.9 63.75) (end 125.9 67.1) (width 0.35) (layer "F.Cu") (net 2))
 (segment (start 127 63.75) (end 127 67.2) (width 0.35) (layer "F.Cu") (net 1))
 (segment (start 127 67.2) (end 127.4 67.6) (width 0.35) (layer "F.Cu") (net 1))
 (segment (start 124.8 54.25) (end 124.8 50.7) (width 0.35) (layer "F.Cu") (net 7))
 (segment (start 124.8 50.7) (end 125.2 50.3) (width 0.35) (layer "F.Cu") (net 7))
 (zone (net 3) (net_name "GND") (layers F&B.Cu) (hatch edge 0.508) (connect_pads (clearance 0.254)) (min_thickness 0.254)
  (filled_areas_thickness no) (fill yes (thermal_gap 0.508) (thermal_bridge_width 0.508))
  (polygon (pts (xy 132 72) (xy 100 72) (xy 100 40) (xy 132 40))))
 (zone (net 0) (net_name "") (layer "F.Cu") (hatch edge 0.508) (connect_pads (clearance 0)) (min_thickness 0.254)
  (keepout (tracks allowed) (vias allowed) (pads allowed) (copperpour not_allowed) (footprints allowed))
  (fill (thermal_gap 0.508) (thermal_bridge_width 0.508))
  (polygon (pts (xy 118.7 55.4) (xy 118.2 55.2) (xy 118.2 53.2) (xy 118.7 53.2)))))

